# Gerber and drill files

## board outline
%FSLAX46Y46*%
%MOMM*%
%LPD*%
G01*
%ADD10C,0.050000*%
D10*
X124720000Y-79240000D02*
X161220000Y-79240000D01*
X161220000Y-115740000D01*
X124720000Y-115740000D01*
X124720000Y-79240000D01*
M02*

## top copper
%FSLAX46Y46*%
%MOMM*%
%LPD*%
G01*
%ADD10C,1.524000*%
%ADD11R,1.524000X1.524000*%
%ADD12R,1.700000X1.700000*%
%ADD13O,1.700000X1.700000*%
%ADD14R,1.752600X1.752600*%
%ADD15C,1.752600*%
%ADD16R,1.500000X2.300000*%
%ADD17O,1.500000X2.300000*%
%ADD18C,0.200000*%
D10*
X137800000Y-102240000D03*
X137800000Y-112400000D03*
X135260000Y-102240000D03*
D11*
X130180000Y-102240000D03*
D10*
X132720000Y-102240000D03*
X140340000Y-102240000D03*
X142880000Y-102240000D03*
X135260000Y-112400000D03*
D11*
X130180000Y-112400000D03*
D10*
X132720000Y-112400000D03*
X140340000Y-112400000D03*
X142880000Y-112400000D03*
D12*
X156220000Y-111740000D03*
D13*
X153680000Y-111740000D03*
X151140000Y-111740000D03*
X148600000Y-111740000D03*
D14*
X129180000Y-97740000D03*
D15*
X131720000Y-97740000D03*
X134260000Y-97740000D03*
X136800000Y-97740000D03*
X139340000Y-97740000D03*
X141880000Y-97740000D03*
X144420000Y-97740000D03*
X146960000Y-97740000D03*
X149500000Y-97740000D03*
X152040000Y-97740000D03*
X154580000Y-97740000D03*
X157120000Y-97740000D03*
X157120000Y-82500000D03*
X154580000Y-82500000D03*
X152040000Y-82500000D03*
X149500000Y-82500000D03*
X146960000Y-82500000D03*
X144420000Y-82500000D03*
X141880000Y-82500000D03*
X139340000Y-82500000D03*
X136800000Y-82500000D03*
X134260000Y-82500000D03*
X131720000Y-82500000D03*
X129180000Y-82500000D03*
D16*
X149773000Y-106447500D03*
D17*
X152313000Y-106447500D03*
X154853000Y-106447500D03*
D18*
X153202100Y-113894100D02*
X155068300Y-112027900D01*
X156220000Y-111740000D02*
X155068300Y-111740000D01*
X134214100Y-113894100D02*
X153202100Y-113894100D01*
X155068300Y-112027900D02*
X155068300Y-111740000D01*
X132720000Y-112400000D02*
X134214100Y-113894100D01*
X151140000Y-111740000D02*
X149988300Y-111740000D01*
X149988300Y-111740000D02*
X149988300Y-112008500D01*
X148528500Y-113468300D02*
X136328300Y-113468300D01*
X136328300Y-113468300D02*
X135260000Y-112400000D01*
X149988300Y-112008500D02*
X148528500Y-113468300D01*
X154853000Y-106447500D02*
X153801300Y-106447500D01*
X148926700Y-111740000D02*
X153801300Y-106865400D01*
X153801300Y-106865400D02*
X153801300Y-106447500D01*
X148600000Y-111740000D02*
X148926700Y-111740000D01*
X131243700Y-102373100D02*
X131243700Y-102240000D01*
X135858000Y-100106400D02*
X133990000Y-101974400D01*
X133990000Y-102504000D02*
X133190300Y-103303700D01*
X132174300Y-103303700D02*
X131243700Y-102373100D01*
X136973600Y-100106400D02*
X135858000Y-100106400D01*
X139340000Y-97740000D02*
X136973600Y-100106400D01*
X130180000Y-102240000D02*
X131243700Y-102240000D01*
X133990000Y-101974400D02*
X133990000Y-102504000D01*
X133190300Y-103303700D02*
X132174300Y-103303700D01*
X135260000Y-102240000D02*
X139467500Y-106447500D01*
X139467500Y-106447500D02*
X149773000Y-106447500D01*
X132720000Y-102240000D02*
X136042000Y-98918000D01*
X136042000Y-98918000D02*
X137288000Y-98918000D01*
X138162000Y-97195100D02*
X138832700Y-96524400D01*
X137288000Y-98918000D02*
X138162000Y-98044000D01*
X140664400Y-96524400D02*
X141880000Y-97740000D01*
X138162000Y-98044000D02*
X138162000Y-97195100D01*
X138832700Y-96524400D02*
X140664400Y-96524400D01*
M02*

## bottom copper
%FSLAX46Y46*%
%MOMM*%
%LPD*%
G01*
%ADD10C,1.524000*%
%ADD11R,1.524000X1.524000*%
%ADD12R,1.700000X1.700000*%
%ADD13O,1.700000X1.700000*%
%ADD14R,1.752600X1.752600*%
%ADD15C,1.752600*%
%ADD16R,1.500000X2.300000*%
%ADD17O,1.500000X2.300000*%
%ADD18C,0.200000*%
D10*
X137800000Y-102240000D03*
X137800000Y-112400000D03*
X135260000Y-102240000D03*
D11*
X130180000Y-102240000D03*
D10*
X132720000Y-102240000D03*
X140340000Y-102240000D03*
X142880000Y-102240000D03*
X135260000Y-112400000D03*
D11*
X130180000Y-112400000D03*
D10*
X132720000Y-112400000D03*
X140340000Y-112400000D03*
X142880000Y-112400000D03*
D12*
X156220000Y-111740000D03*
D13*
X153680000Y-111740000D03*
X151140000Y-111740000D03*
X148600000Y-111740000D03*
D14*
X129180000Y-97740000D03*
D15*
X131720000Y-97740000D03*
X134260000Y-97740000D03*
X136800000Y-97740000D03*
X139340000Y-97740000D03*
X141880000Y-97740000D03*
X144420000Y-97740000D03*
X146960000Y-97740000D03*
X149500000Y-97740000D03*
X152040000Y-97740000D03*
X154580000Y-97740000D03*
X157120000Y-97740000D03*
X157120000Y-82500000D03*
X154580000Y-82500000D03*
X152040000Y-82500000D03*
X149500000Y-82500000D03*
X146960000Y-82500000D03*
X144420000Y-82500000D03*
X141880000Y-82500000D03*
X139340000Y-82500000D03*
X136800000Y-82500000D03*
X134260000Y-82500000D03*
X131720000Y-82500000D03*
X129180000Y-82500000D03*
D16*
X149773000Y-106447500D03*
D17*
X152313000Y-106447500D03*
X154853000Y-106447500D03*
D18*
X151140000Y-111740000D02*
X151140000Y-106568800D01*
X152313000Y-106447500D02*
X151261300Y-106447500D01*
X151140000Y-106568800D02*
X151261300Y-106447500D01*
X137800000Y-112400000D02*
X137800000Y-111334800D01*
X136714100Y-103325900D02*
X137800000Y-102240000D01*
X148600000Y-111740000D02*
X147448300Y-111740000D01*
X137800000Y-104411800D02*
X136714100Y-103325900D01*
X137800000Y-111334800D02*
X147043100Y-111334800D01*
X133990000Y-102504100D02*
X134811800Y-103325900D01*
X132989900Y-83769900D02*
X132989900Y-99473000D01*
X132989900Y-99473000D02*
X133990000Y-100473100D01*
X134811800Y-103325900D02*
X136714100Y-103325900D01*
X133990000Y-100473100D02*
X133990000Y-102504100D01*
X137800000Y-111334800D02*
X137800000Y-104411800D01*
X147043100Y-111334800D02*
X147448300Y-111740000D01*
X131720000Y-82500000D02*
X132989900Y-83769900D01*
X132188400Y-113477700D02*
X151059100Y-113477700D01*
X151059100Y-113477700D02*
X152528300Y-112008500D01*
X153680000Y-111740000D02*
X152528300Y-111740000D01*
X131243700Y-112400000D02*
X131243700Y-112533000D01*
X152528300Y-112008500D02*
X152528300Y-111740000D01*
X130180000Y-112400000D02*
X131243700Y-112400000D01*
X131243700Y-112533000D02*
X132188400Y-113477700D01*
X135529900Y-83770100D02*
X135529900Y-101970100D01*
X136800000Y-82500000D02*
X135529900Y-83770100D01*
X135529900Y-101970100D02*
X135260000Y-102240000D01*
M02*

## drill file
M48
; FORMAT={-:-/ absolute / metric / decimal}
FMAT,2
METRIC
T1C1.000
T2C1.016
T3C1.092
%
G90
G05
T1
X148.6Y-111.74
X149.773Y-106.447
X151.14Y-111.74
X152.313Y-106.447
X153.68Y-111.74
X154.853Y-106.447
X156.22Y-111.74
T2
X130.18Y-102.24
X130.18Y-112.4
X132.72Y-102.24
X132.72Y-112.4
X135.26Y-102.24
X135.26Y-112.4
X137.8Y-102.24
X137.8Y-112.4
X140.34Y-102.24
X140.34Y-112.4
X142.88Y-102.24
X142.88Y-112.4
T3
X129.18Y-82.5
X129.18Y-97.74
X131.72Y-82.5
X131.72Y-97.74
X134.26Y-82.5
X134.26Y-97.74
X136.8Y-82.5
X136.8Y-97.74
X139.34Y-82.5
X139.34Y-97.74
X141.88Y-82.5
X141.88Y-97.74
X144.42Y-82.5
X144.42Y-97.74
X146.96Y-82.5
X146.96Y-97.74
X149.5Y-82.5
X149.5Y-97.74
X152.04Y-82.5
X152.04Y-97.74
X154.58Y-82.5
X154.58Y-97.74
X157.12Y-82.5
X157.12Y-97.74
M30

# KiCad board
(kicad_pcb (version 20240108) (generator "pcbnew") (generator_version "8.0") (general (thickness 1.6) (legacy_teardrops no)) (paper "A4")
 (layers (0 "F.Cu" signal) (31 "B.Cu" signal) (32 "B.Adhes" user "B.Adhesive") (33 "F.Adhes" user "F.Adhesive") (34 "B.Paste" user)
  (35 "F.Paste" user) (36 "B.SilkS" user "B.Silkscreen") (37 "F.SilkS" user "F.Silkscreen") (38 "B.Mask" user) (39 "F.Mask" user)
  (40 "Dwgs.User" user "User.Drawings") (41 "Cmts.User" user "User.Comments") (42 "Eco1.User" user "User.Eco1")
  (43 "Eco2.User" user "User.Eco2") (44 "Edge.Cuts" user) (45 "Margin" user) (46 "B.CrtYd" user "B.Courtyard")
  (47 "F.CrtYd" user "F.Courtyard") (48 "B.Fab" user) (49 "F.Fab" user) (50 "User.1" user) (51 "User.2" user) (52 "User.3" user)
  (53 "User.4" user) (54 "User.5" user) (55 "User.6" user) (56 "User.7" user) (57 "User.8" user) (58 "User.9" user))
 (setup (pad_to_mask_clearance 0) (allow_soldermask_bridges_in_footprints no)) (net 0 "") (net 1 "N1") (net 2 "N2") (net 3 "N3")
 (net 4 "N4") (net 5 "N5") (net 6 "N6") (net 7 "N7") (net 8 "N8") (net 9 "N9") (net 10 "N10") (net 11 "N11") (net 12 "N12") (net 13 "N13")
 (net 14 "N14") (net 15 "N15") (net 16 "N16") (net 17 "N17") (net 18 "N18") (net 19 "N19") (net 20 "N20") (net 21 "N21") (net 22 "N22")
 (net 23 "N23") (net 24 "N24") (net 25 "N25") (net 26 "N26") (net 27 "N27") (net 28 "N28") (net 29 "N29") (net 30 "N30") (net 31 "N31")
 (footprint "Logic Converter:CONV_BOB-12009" (layer "F.Cu") (at 136.53 107.32 90)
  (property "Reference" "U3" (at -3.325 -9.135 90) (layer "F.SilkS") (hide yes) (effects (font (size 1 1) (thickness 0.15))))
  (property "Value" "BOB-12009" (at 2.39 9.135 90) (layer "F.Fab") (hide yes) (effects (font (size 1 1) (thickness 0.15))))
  (pad "GND_1" thru_hole circle (at 5.08 1.27 90) (size 1.524 1.524) (drill 1.016) (layers "*.Cu" "*.Mask") (remove_unused_layers no)
   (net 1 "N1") (solder_mask_margin 0.102))
  (pad "GND_2" thru_hole circle (at -5.08 1.27 90) (size 1.524 1.524) (drill 1.016) (layers "*.Cu" "*.Mask") (remove_unused_layers no)
   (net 1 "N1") (solder_mask_margin 0.102))
  (pad "HV" thru_hole circle (at 5.08 -1.27 90) (size 1.524 1.524) (drill 1.016) (layers "*.Cu" "*.Mask") (remove_unused_layers no)
   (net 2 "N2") (solder_mask_margin 0.102))
  (pad "HV1" thru_hole rect (at 5.08 -6.35 90) (size 1.524 1.524) (drill 1.016) (layers "*.Cu" "*.Mask") (remove_unused_layers no)
   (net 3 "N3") (solder_mask_margin 0.102))
  (pad "HV2" thru_hole circle (at 5.08 -3.81 90) (size 1.524 1.524) (drill 1.016) (layers "*.Cu" "*.Mask") (remove_unused_layers no)
   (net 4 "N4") (solder_mask_margin 0.102))
  (pad "HV3" thru_hole circle (at 5.08 3.81 90) (size 1.524 1.524) (drill 1.016) (layers "*.Cu" "*.Mask") (remove_unused_layers no)
   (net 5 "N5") (solder_mask_margin 0.102))
  (pad "HV4" thru_hole circle (at 5.08 6.35 90) (size 1.524 1.524) (drill 1.016) (layers "*.Cu" "*.Mask") (remove_unused_layers no)
   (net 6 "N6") (solder_mask_margin 0.102))
  (pad "LV" thru_hole circle (at -5.08 -1.27 90) (size 1.524 1.524) (drill 1.016) (layers "*.Cu" "*.Mask") (remove_unused_layers no)
   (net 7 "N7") (solder_mask_margin 0.102))
  (pad "LV1" thru_hole rect (at -5.08 -6.35 90) (size 1.524 1.524) (drill 1.016) (layers "*.Cu" "*.Mask") (remove_unused_layers no)
   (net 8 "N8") (solder_mask_margin 0.102))
  (pad "LV2" thru_hole circle (at -5.08 -3.81 90) (size 1.524 1.524) (drill 1.016) (layers "*.Cu" "*.Mask") (remove_unused_layers no)
   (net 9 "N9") (solder_mask_margin 0.102))
  (pad "LV3" thru_hole circle (at -5.08 3.81 90) (size 1.524 1.524) (drill 1.016) (layers "*.Cu" "*.Mask") (remove_unused_layers no)
   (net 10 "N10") (solder_mask_margin 0.102))
  (pad "LV4" thru_hole circle (at -5.08 6.35 90) (size 1.524 1.524) (drill 1.016) (layers "*.Cu" "*.Mask") (remove_unused_layers no)
   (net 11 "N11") (solder_mask_margin 0.102)))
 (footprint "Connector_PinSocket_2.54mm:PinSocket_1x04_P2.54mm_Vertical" (layer "F.Cu") (at 156.22 111.74 -90)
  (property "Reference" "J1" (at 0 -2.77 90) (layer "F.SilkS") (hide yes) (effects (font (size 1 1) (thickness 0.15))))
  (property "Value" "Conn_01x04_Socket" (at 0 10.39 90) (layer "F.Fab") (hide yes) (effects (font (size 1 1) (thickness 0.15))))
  (pad "1" thru_hole rect (at 0 0 270) (size 1.7 1.7) (drill 1) (layers "*.Cu" "*.Mask") (remove_unused_layers no) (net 9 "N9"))
  (pad "2" thru_hole oval (at 0 2.54 270) (size 1.7 1.7) (drill 1) (layers "*.Cu" "*.Mask") (remove_unused_layers no) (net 8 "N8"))
  (pad "3" thru_hole oval (at 0 5.08 270) (size 1.7 1.7) (drill 1) (layers "*.Cu" "*.Mask") (remove_unused_layers no) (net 7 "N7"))
  (pad "4" thru_hole oval (at 0 7.62 270) (size 1.7 1.7) (drill 1) (layers "*.Cu" "*.Mask") (remove_unused_layers no) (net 1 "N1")))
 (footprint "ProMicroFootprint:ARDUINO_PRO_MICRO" (layer "F.Cu") (at 143.15 90.12)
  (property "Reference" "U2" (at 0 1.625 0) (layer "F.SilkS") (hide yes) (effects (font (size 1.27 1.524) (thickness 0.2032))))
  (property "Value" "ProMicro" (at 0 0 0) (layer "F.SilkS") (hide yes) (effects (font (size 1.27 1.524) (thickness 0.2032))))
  (pad "1" thru_hole rect (at -13.97 7.62) (size 1.7526 1.7526) (drill 1.0922) (layers "*.Cu" "*.SilkS" "*.Mask") (remove_unused_layers no)
   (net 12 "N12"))
  (pad "2" thru_hole circle (at -11.43 7.62) (size 1.7526 1.7526) (drill 1.0922) (layers "*.Cu" "*.SilkS" "*.Mask")
   (remove_unused_layers no) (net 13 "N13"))
  (pad "3" thru_hole circle (at -8.89 7.62) (size 1.7526 1.7526) (drill 1.0922) (layers "*.Cu" "*.SilkS" "*.Mask") (remove_unused_layers no)
   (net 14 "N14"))
  (pad "4" thru_hole circle (at -6.35 7.62) (size 1.7526 1.7526) (drill 1.0922) (layers "*.Cu" "*.SilkS" "*.Mask") (remove_unused_layers no)
   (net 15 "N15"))
  (pad "5" thru_hole circle (at -3.81 7.62) (size 1.7526 1.7526) (drill 1.0922) (layers "*.Cu" "*.SilkS" "*.Mask") (remove_unused_layers no)
   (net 3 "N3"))
  (pad "6" thru_hole circle (at -1.27 7.62) (size 1.7526 1.7526) (drill 1.0922) (layers "*.Cu" "*.SilkS" "*.Mask") (remove_unused_layers no)
   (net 4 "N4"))
  (pad "7" thru_hole circle (at 1.27 7.62) (size 1.7526 1.7526) (drill 1.0922) (layers "*.Cu" "*.SilkS" "*.Mask") (remove_unused_layers no)
   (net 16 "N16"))
  (pad "8" thru_hole circle (at 3.81 7.62) (size 1.7526 1.7526) (drill 1.0922) (layers "*.Cu" "*.SilkS" "*.Mask") (remove_unused_layers no)
   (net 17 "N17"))
  (pad "9" thru_hole circle (at 6.35 7.62) (size 1.7526 1.7526) (drill 1.0922) (layers "*.Cu" "*.SilkS" "*.Mask") (remove_unused_layers no)
   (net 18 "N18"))
  (pad "10" thru_hole circle (at 8.89 7.62) (size 1.7526 1.7526) (drill 1.0922) (layers "*.Cu" "*.SilkS" "*.Mask") (remove_unused_layers no)
   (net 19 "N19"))
  (pad "11" thru_hole circle (at 11.43 7.62) (size 1.7526 1.7526) (drill 1.0922) (layers "*.Cu" "*.SilkS" "*.Mask")
   (remove_unused_layers no) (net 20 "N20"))
  (pad "12" thru_hole circle (at 13.97 7.62) (size 1.7526 1.7526) (drill 1.0922) (layers "*.Cu" "*.SilkS" "*.Mask")
   (remove_unused_layers no) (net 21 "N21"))
  (pad "13" thru_hole circle (at 13.97 -7.62) (size 1.7526 1.7526) (drill 1.0922) (layers "*.Cu" "*.SilkS" "*.Mask")
   (remove_unused_layers no) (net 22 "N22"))
  (pad "14" thru_hole circle (at 11.43 -7.62) (size 1.7526 1.7526) (drill 1.0922) (layers "*.Cu" "*.SilkS" "*.Mask")
   (remove_unused_layers no) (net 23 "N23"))
  (pad "15" thru_hole circle (at 8.89 -7.62) (size 1.7526 1.7526) (drill 1.0922) (layers "*.Cu" "*.SilkS" "*.Mask")
   (remove_unused_layers no) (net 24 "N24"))
  (pad "16" thru_hole circle (at 6.35 -7.62) (size 1.7526 1.7526) (drill 1.0922) (layers "*.Cu" "*.SilkS" "*.Mask")
   (remove_unused_layers no) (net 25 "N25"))
  (pad "17" thru_hole circle (at 3.81 -7.62) (size 1.7526 1.7526) (drill 1.0922) (layers "*.Cu" "*.SilkS" "*.Mask")
   (remove_unused_layers no) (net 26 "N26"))
  (pad "18" thru_hole circle (at 1.27 -7.62) (size 1.7526 1.7526) (drill 1.0922) (layers "*.Cu" "*.SilkS" "*.Mask")
   (remove_unused_layers no) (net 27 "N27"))
  (pad "19" thru_hole circle (at -1.27 -7.62) (size 1.7526 1.7526) (drill 1.0922) (layers "*.Cu" "*.SilkS" "*.Mask")
   (remove_unused_layers no) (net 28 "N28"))
  (pad "20" thru_hole circle (at -3.81 -7.62) (size 1.7526 1.7526) (drill 1.0922) (layers "*.Cu" "*.SilkS" "*.Mask")
   (remove_unused_layers no) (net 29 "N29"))
  (pad "21" thru_hole circle (at -6.35 -7.62) (size 1.7526 1.7526) (drill 1.0922) (layers "*.Cu" "*.SilkS" "*.Mask")
   (remove_unused_layers no) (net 2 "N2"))
  (pad "22" thru_hole circle (at -8.89 -7.62) (size 1.7526 1.7526) (drill 1.0922) (layers "*.Cu" "*.SilkS" "*.Mask")
   (remove_unused_layers no) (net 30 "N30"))
  (pad "23" thru_hole circle (at -11.43 -7.62) (size 1.7526 1.7526) (drill 1.0922) (layers "*.Cu" "*.SilkS" "*.Mask")
   (remove_unused_layers no) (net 1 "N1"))
  (pad "24" thru_hole circle (at -13.97 -7.62) (size 1.7526 1.7526) (drill 1.0922) (layers "*.Cu" "*.SilkS" "*.Mask")
   (remove_unused_layers no) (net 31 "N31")))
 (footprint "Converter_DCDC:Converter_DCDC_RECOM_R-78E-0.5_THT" (layer "F.Cu") (at 149.773 106.4475)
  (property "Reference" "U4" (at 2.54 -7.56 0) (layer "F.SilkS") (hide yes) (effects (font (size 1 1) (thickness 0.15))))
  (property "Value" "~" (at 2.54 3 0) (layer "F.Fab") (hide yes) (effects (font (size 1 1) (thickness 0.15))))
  (pad "1" thru_hole rect (at 0 0) (size 1.5 2.3) (drill 1) (layers "*.Cu" "*.Mask") (remove_unused_layers no) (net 2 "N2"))
  (pad "2" thru_hole oval (at 2.54 0) (size 1.5 2.3) (drill 1) (layers "*.Cu" "*.Mask") (remove_unused_layers no) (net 7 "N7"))
  (pad "3" thru_hole oval (at 5.08 0) (size 1.5 2.3) (drill 1) (layers "*.Cu" "*.Mask") (remove_unused_layers no) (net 1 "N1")))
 (gr_rect (start 124.72 79.24) (end 161.22 115.74) (stroke (width 0.05) (type default)) (fill none) (layer "Edge.Cuts"))
 (segment (start 153.2021 113.8941) (end 155.0683 112.0279) (width 0.2) (layer "F.Cu") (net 9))
 (segment (start 156.22 111.74) (end 155.0683 111.74) (width 0.2) (layer "F.Cu") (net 9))
 (segment (start 134.2141 113.8941) (end 153.2021 113.8941) (width 0.2) (layer "F.Cu") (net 9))
 (segment (start 155.0683 112.0279) (end 155.0683 111.74) (width 0.2) (layer "F.Cu") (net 9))
 (segment (start 132.72 112.4) (end 134.2141 113.8941) (width 0.2) (layer "F.Cu") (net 9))
 (segment (start 151.14 111.74) (end 149.9883 111.74) (width 0.2) (layer "F.Cu") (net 7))
 (segment (start 149.9883 111.74) (end 149.9883 112.0085) (width 0.2) (layer "F.Cu") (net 7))
 (segment (start 148.5285 113.4683) (end 136.3283 113.4683) (width 0.2) (layer "F.Cu") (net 7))
 (segment (start 136.3283 113.4683) (end 135.26 112.4) (width 0.2) (layer "F.Cu") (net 7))
 (segment (start 149.9883 112.0085) (end 148.5285 113.4683) (width 0.2) (layer "F.Cu") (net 7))
 (segment (start 151.14 111.74) (end 151.14 106.5688) (width 0.2) (layer "B.Cu") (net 7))
 (segment (start 152.313 106.4475) (end 151.2613 106.4475) (width 0.2) (layer "B.Cu") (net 7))
 (segment (start 151.14 106.5688) (end 151.2613 106.4475) (width 0.2) (layer "B.Cu") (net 7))
 (segment (start 154.853 106.4475) (end 153.8013 106.4475) (width 0.2) (layer "F.Cu") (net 1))
 (segment (start 148.9267 111.74) (end 153.8013 106.8654) (width 0.2) (layer "F.Cu") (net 1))
 (segment (start 153.8013 106.8654) (end 153.8013 106.4475) (width 0.2) (layer "F.Cu") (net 1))
 (segment (start 148.6 111.74) (end 148.9267 111.74) (width 0.2) (layer "F.Cu") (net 1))
 (segment (start 137.8 112.4) (end 137.8 111.3348) (width 0.2) (layer "B.Cu") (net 1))
 (segment (start 136.7141 103.3259) (end 137.8 102.24) (width 0.2) (layer "B.Cu") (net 1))
 (segment (start 148.6 111.74) (end 147.4483 111.74) (width 0.2) (layer "B.Cu") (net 1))
 (segment (start 137.8 104.4118) (end 136.7141 103.3259) (width 0.2) (layer "B.Cu") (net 1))
 (segment (start 137.8 111.3348) (end 147.0431 111.3348) (width 0.2) (layer "B.Cu") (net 1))
 (segment (start 133.99 102.5041) (end 134.8118 103.3259) (width 0.2) (layer "B.Cu") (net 1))
 (segment (start 132.9899 83.7699) (end 132.9899 99.473) (width 0.2) (layer "B.Cu") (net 1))
 (segment (start 132.9899 99.473) (end 133.99 100.4731) (width 0.2) (layer "B.Cu") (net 1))
 (segment (start 134.8118 103.3259) (end 136.7141 103.3259) (width 0.2) (layer "B.Cu") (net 1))
 (segment (start 133.99 100.4731) (end 133.99 102.5041) (width 0.2) (layer "B.Cu") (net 1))
 (segment (start 137.8 111.3348) (end 137.8 104.4118) (width 0.2) (layer "B.Cu") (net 1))
 (segment (start 147.0431 111.3348) (end 147.4483 111.74) (width 0.2) (layer "B.Cu") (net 1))
 (segment (start 131.72 82.5) (end 132.9899 83.7699) (width 0.2) (layer "B.Cu") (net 1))
 (segment (start 132.1884 113.4777) (end 151.0591 113.4777) (width 0.2) (layer "B.Cu") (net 8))
 (segment (start 151.0591 113.4777) (end 152.5283 112.0085) (width 0.2) (layer "B.Cu") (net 8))
 (segment (start 153.68 111.74) (end 152.5283 111.74) (width 0.2) (layer "B.Cu") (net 8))
 (segment (start 131.2437 112.4) (end 131.2437 112.533) (width 0.2) (layer "B.Cu") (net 8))
 (segment (start 152.5283 112.0085) (end 152.5283 111.74) (width 0.2) (layer "B.Cu") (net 8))
 (segment (start 130.18 112.4) (end 131.2437 112.4) (width 0.2) (layer "B.Cu") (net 8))
 (segment (start 131.2437 112.533) (end 132.1884 113.4777) (width 0.2) (layer "B.Cu") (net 8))
 (segment (start 131.2437 102.3731) (end 131.2437 102.24) (width 0.2) (layer "F.Cu") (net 3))
 (segment (start 135.858 100.1064) (end 133.99 101.9744) (width 0.2) (layer "F.Cu") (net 3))
 (segment (start 133.99 102.504) (end 133.1903 103.3037) (width 0.2) (layer "F.Cu") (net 3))
 (segment (start 132.1743 103.3037) (end 131.2437 102.3731) (width 0.2) (layer "F.Cu") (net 3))
 (segment (start 136.9736 100.1064) (end 135.858 100.1064) (width 0.2) (layer "F.Cu") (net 3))
 (segment (start 139.34 97.74) (end 136.9736 100.1064) (width 0.2) (layer "F.Cu") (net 3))
 (segment (start 130.18 102.24) (end 131.2437 102.24) (width 0.2) (layer "F.Cu") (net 3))
 (segment (start 133.99 101.9744) (end 133.99 102.504) (width 0.2) (layer "F.Cu") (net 3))
 (segment (start 133.1903 103.3037) (end 132.1743 103.3037) (width 0.2) (layer "F.Cu") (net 3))
 (segment (start 135.26 102.24) (end 139.4675 106.4475) (width 0.2) (layer "F.Cu") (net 2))
 (segment (start 139.4675 106.4475) (end 149.773 106.4475) (width 0.2) (layer "F.Cu") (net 2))
 (segment (start 135.5299 83.7701) (end 135.5299 101.9701) (width 0.2) (layer "B.Cu") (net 2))
 (segment (start 136.8 82.5) (end 135.5299 83.7701) (width 0.2) (layer "B.Cu") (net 2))
 (segment (start 135.5299 101.9701) (end 135.26 102.24) (width 0.2) (layer "B.Cu") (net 2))
 (segment (start 132.72 102.24) (end 136.042 98.918) (width 0.2) (layer "F.Cu") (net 4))
 (segment (start 136.042 98.918) (end 137.288 98.918) (width 0.2) (layer "F.Cu") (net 4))
 (segment (start 138.162 97.1951) (end 138.8327 96.5244) (width 0.2) (layer "F.Cu") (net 4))
 (segment (start 137.288 98.918) (end 138.162 98.044) (width 0.2) (layer "F.Cu") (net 4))
 (segment (start 140.6644 96.5244) (end 141.88 97.74) (width 0.2) (layer "F.Cu") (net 4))
 (segment (start 138.162 98.044) (end 138.162 97.1951) (width 0.2) (layer "F.Cu") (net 4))
 (segment (start 138.8327 96.5244) (end 140.6644 96.5244) (width 0.2) (layer "F.Cu") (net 4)))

